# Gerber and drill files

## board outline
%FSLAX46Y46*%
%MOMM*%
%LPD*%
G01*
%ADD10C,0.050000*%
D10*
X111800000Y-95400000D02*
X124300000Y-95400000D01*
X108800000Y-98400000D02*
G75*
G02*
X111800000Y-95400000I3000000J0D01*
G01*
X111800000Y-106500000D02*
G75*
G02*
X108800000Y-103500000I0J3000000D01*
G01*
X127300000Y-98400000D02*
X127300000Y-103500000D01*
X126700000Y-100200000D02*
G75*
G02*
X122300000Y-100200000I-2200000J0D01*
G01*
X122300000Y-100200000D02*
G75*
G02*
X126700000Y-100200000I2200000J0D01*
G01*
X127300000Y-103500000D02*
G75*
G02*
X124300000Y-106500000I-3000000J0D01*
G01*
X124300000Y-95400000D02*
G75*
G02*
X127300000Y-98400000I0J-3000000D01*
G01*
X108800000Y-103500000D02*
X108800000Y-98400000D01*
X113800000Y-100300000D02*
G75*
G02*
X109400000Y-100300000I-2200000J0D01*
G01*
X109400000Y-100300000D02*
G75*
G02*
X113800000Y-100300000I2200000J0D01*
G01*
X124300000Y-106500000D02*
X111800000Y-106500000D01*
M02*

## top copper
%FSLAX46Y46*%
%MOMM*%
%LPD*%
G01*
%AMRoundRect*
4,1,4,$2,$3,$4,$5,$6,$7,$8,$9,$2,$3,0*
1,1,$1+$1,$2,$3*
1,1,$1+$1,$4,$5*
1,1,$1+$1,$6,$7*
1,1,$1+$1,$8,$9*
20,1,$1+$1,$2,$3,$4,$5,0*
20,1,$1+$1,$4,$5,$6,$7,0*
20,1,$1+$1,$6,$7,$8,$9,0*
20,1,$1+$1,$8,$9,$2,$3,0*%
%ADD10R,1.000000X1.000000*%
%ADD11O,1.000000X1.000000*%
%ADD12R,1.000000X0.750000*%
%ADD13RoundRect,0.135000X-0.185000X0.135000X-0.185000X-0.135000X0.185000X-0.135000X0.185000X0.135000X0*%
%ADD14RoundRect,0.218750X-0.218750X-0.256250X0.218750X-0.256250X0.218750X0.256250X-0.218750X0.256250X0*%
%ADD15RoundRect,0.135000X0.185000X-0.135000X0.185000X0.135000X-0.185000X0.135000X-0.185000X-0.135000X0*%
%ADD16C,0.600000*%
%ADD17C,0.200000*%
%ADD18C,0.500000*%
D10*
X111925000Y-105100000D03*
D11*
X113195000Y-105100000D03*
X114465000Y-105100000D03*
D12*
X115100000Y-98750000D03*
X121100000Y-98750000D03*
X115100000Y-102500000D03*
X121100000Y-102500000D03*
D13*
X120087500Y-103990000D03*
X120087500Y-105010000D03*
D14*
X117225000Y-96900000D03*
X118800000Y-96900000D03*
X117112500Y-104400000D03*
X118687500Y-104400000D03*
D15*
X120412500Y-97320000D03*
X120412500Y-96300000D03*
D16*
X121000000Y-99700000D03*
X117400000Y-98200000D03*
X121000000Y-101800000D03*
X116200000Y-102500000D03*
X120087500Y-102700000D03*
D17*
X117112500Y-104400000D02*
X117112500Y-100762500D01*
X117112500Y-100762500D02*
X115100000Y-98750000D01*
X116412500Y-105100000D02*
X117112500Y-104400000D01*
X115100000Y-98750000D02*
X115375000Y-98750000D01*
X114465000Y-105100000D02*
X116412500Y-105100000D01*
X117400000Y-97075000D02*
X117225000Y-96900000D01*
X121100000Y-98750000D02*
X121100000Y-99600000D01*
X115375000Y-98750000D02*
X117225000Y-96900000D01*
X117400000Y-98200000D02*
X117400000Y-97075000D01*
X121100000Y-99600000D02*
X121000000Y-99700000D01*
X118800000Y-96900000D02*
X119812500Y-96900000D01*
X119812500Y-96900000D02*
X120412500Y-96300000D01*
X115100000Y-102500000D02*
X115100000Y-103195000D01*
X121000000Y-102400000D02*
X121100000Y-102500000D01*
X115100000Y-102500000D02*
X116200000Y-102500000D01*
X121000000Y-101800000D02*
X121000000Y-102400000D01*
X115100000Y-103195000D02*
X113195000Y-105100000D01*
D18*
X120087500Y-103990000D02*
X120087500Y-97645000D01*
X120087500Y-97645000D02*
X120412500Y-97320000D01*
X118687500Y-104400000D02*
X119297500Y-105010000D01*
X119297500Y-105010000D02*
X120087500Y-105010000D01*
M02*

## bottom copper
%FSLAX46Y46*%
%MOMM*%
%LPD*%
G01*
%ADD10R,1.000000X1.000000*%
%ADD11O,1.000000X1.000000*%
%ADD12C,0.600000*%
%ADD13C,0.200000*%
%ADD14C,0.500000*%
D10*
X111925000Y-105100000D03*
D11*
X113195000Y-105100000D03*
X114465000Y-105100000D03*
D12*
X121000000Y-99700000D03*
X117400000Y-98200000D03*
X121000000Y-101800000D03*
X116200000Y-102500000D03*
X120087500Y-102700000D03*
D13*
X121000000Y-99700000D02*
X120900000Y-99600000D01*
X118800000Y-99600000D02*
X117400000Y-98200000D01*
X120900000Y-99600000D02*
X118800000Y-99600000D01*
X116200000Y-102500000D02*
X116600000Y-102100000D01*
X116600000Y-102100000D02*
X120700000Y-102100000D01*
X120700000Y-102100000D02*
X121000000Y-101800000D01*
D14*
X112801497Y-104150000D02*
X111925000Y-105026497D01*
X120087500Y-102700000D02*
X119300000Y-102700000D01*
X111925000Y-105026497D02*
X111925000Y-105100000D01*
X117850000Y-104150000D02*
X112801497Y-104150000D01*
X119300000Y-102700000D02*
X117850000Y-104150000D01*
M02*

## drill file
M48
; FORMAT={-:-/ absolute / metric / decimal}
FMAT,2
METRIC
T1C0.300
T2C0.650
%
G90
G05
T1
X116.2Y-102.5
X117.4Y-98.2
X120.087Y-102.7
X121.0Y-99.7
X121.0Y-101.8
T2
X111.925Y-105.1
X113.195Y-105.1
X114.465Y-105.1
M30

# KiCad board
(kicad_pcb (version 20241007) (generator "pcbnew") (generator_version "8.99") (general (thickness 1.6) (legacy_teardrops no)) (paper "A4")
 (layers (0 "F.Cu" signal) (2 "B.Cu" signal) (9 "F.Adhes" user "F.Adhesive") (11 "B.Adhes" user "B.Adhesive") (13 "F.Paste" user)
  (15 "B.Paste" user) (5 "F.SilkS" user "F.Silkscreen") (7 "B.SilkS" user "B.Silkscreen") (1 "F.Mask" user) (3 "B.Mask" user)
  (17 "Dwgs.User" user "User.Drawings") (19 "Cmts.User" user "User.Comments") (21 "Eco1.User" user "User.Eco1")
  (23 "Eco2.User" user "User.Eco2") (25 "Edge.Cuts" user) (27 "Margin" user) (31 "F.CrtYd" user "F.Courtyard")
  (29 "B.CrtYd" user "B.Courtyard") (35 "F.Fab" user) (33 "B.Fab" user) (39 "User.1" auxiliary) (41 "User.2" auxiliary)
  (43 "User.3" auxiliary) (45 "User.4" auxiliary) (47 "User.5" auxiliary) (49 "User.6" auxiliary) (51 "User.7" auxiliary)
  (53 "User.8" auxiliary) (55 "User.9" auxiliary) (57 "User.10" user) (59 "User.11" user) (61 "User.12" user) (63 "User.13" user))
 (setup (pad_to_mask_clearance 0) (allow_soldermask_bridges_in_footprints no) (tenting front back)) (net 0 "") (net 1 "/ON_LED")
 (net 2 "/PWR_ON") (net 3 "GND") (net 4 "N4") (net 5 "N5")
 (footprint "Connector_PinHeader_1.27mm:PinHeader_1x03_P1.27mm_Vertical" (layer "F.Cu") (at 111.925 105.1 90)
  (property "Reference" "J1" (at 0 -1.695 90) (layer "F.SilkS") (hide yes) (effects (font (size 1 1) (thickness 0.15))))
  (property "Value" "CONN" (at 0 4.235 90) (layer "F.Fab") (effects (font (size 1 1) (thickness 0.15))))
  (pad "1" thru_hole rect (at 0 0 90) (size 1 1) (drill 0.65) (layers "*.Cu" "*.Mask") (remove_unused_layers no) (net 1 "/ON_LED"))
  (pad "2" thru_hole oval (at 0 1.27 90) (size 1 1) (drill 0.65) (layers "*.Cu" "*.Mask") (remove_unused_layers no) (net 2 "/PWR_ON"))
  (pad "3" thru_hole oval (at 0 2.54 90) (size 1 1) (drill 0.65) (layers "*.Cu" "*.Mask") (remove_unused_layers no) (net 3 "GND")))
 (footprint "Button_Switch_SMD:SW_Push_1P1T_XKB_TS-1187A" (layer "F.Cu") (at 118.1 100.625)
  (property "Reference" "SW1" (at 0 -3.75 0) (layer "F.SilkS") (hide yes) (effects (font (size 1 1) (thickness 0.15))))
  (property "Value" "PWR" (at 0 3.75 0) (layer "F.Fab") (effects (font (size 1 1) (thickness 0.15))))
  (pad "1" smd rect (at -3 -1.875) (size 1 0.75) (layers "F.Cu" "F.Mask" "F.Paste") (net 3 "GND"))
  (pad "1" smd rect (at 3 -1.875) (size 1 0.75) (layers "F.Cu" "F.Mask" "F.Paste") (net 3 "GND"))
  (pad "2" smd rect (at -3 1.875) (size 1 0.75) (layers "F.Cu" "F.Mask" "F.Paste") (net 2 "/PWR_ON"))
  (pad "2" smd rect (at 3 1.875) (size 1 0.75) (layers "F.Cu" "F.Mask" "F.Paste") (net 2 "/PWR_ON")))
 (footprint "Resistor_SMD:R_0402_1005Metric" (layer "F.Cu") (at 120.0875 104.5 -90)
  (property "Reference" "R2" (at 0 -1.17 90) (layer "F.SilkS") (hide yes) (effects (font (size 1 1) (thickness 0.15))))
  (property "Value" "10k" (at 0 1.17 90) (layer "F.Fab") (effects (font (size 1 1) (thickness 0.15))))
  (pad "1" smd roundrect (at -0.51 0 270) (size 0.54 0.64) (layers "F.Cu" "F.Mask" "F.Paste") (roundrect_rratio 0.25) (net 1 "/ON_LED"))
  (pad "2" smd roundrect (at 0.51 0 270) (size 0.54 0.64) (layers "F.Cu" "F.Mask" "F.Paste") (roundrect_rratio 0.25) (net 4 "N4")))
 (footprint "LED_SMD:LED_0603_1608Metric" (layer "F.Cu") (at 118.0125 96.9)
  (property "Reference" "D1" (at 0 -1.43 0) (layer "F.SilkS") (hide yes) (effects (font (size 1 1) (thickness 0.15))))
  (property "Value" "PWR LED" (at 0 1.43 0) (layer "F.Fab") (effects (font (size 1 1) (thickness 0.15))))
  (pad "1" smd roundrect (at -0.7875 0) (size 0.875 0.95) (layers "F.Cu" "F.Mask" "F.Paste") (roundrect_rratio 0.25) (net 3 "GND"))
  (pad "2" smd roundrect (at 0.7875 0) (size 0.875 0.95) (layers "F.Cu" "F.Mask" "F.Paste") (roundrect_rratio 0.25) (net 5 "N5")))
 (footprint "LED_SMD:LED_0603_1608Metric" (layer "F.Cu") (at 117.9 104.4)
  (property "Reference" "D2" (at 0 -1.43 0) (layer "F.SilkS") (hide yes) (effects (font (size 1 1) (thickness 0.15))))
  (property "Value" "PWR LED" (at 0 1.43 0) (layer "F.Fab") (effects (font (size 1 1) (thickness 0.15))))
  (pad "1" smd roundrect (at -0.7875 0) (size 0.875 0.95) (layers "F.Cu" "F.Mask" "F.Paste") (roundrect_rratio 0.25) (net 3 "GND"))
  (pad "2" smd roundrect (at 0.7875 0) (size 0.875 0.95) (layers "F.Cu" "F.Mask" "F.Paste") (roundrect_rratio 0.25) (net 4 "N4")))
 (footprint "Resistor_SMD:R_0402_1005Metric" (layer "F.Cu") (at 120.4125 96.81 90)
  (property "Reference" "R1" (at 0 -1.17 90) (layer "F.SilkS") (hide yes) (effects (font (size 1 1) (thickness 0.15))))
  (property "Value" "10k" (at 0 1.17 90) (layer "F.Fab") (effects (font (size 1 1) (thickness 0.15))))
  (pad "1" smd roundrect (at -0.51 0 90) (size 0.54 0.64) (layers "F.Cu" "F.Mask" "F.Paste") (roundrect_rratio 0.25) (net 1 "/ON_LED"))
  (pad "2" smd roundrect (at 0.51 0 90) (size 0.54 0.64) (layers "F.Cu" "F.Mask" "F.Paste") (roundrect_rratio 0.25) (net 5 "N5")))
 (gr_line (start 111.8 95.4) (end 124.3 95.4) (stroke (width 0.05) (type default)) (layer "Edge.Cuts"))
 (gr_arc (start 108.8 98.4) (mid 109.67868 96.27868) (end 111.8 95.4) (stroke (width 0.05) (type default)) (layer "Edge.Cuts"))
 (gr_arc (start 111.8 106.5) (mid 109.67868 105.62132) (end 108.8 103.5) (stroke (width 0.05) (type default)) (layer "Edge.Cuts"))
 (gr_line (start 127.3 98.4) (end 127.3 103.5) (stroke (width 0.05) (type default)) (layer "Edge.Cuts"))
 (gr_circle (center 124.5 100.2) (end 126.7 100.2) (stroke (width 0.05) (type default)) (fill none) (layer "Edge.Cuts"))
 (gr_arc (start 127.3 103.5) (mid 126.42132 105.62132) (end 124.3 106.5) (stroke (width 0.05) (type default)) (layer "Edge.Cuts"))
 (gr_arc (start 124.3 95.4) (mid 126.42132 96.27868) (end 127.3 98.4) (stroke (width 0.05) (type default)) (layer "Edge.Cuts"))
 (gr_line (start 108.8 103.5) (end 108.8 98.4) (stroke (width 0.05) (type default)) (layer "Edge.Cuts"))
 (gr_circle (center 111.6 100.3) (end 113.8 100.3) (stroke (width 0.05) (type default)) (fill none) (layer "Edge.Cuts"))
 (gr_line (start 124.3 106.5) (end 111.8 106.5) (stroke (width 0.05) (type default)) (layer "Edge.Cuts"))
 (segment (start 117.1125 104.4) (end 117.1125 100.7625) (width 0.2) (layer "F.Cu") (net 3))
 (segment (start 117.1125 100.7625) (end 115.1 98.75) (width 0.2) (layer "F.Cu") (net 3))
 (segment (start 116.4125 105.1) (end 117.1125 104.4) (width 0.2) (layer "F.Cu") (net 3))
 (segment (start 115.1 98.75) (end 115.375 98.75) (width 0.2) (layer "F.Cu") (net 3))
 (segment (start 114.465 105.1) (end 116.4125 105.1) (width 0.2) (layer "F.Cu") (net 3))
 (segment (start 117.4 97.075) (end 117.225 96.9) (width 0.2) (layer "F.Cu") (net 3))
 (segment (start 121.1 98.75) (end 121.1 99.6) (width 0.2) (layer "F.Cu") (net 3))
 (segment (start 115.375 98.75) (end 117.225 96.9) (width 0.2) (layer "F.Cu") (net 3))
 (segment (start 117.4 98.2) (end 117.4 97.075) (width 0.2) (layer "F.Cu") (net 3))
 (segment (start 121.1 99.6) (end 121 99.7) (width 0.2) (layer "F.Cu") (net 3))
 (via (at 121 99.7) (size 0.6) (drill 0.3) (layers "F.Cu" "B.Cu") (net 3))
 (via (at 117.4 98.2) (size 0.6) (drill 0.3) (layers "F.Cu" "B.Cu") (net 3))
 (segment (start 121 99.7) (end 120.9 99.6) (width 0.2) (layer "B.Cu") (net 3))
 (segment (start 118.8 99.6) (end 117.4 98.2) (width 0.2) (layer "B.Cu") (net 3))
 (segment (start 120.9 99.6) (end 118.8 99.6) (width 0.2) (layer "B.Cu") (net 3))
 (segment (start 118.8 96.9) (end 119.8125 96.9) (width 0.2) (layer "F.Cu") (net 5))
 (segment (start 119.8125 96.9) (end 120.4125 96.3) (width 0.2) (layer "F.Cu") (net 5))
 (segment (start 115.1 102.5) (end 115.1 103.195) (width 0.2) (layer "F.Cu") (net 2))
 (segment (start 121 102.4) (end 121.1 102.5) (width 0.2) (layer "F.Cu") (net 2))
 (segment (start 115.1 102.5) (end 116.2 102.5) (width 0.2) (layer "F.Cu") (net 2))
 (segment (start 121 101.8) (end 121 102.4) (width 0.2) (layer "F.Cu") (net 2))
 (segment (start 115.1 103.195) (end 113.195 105.1) (width 0.2) (layer "F.Cu") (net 2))
 (via (at 121 101.8) (size 0.6) (drill 0.3) (layers "F.Cu" "B.Cu") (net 2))
 (via (at 116.2 102.5) (size 0.6) (drill 0.3) (layers "F.Cu" "B.Cu") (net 2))
 (segment (start 116.2 102.5) (end 116.6 102.1) (width 0.2) (layer "B.Cu") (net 2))
 (segment (start 116.6 102.1) (end 120.7 102.1) (width 0.2) (layer "B.Cu") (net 2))
 (segment (start 120.7 102.1) (end 121 101.8) (width 0.2) (layer "B.Cu") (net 2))
 (segment (start 120.0875 103.99) (end 120.0875 97.645) (width 0.5) (layer "F.Cu") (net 1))
 (segment (start 120.0875 97.645) (end 120.4125 97.32) (width 0.5) (layer "F.Cu") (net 1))
 (via (at 120.0875 102.7) (size 0.6) (drill 0.3) (layers "F.Cu" "B.Cu") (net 1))
 (segment (start 112.801497 104.15) (end 111.925 105.026497) (width 0.5) (layer "B.Cu") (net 1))
 (segment (start 120.0875 102.7) (end 119.3 102.7) (width 0.5) (layer "B.Cu") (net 1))
 (segment (start 111.925 105.026497) (end 111.925 105.1) (width 0.5) (layer "B.Cu") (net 1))
 (segment (start 117.85 104.15) (end 112.801497 104.15) (width 0.5) (layer "B.Cu") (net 1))
 (segment (start 119.3 102.7) (end 117.85 104.15) (width 0.5) (layer "B.Cu") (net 1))
 (segment (start 118.6875 104.4) (end 119.2975 105.01) (width 0.5) (layer "F.Cu") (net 4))
 (segment (start 119.2975 105.01) (end 120.0875 105.01) (width 0.5) (layer "F.Cu") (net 4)))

